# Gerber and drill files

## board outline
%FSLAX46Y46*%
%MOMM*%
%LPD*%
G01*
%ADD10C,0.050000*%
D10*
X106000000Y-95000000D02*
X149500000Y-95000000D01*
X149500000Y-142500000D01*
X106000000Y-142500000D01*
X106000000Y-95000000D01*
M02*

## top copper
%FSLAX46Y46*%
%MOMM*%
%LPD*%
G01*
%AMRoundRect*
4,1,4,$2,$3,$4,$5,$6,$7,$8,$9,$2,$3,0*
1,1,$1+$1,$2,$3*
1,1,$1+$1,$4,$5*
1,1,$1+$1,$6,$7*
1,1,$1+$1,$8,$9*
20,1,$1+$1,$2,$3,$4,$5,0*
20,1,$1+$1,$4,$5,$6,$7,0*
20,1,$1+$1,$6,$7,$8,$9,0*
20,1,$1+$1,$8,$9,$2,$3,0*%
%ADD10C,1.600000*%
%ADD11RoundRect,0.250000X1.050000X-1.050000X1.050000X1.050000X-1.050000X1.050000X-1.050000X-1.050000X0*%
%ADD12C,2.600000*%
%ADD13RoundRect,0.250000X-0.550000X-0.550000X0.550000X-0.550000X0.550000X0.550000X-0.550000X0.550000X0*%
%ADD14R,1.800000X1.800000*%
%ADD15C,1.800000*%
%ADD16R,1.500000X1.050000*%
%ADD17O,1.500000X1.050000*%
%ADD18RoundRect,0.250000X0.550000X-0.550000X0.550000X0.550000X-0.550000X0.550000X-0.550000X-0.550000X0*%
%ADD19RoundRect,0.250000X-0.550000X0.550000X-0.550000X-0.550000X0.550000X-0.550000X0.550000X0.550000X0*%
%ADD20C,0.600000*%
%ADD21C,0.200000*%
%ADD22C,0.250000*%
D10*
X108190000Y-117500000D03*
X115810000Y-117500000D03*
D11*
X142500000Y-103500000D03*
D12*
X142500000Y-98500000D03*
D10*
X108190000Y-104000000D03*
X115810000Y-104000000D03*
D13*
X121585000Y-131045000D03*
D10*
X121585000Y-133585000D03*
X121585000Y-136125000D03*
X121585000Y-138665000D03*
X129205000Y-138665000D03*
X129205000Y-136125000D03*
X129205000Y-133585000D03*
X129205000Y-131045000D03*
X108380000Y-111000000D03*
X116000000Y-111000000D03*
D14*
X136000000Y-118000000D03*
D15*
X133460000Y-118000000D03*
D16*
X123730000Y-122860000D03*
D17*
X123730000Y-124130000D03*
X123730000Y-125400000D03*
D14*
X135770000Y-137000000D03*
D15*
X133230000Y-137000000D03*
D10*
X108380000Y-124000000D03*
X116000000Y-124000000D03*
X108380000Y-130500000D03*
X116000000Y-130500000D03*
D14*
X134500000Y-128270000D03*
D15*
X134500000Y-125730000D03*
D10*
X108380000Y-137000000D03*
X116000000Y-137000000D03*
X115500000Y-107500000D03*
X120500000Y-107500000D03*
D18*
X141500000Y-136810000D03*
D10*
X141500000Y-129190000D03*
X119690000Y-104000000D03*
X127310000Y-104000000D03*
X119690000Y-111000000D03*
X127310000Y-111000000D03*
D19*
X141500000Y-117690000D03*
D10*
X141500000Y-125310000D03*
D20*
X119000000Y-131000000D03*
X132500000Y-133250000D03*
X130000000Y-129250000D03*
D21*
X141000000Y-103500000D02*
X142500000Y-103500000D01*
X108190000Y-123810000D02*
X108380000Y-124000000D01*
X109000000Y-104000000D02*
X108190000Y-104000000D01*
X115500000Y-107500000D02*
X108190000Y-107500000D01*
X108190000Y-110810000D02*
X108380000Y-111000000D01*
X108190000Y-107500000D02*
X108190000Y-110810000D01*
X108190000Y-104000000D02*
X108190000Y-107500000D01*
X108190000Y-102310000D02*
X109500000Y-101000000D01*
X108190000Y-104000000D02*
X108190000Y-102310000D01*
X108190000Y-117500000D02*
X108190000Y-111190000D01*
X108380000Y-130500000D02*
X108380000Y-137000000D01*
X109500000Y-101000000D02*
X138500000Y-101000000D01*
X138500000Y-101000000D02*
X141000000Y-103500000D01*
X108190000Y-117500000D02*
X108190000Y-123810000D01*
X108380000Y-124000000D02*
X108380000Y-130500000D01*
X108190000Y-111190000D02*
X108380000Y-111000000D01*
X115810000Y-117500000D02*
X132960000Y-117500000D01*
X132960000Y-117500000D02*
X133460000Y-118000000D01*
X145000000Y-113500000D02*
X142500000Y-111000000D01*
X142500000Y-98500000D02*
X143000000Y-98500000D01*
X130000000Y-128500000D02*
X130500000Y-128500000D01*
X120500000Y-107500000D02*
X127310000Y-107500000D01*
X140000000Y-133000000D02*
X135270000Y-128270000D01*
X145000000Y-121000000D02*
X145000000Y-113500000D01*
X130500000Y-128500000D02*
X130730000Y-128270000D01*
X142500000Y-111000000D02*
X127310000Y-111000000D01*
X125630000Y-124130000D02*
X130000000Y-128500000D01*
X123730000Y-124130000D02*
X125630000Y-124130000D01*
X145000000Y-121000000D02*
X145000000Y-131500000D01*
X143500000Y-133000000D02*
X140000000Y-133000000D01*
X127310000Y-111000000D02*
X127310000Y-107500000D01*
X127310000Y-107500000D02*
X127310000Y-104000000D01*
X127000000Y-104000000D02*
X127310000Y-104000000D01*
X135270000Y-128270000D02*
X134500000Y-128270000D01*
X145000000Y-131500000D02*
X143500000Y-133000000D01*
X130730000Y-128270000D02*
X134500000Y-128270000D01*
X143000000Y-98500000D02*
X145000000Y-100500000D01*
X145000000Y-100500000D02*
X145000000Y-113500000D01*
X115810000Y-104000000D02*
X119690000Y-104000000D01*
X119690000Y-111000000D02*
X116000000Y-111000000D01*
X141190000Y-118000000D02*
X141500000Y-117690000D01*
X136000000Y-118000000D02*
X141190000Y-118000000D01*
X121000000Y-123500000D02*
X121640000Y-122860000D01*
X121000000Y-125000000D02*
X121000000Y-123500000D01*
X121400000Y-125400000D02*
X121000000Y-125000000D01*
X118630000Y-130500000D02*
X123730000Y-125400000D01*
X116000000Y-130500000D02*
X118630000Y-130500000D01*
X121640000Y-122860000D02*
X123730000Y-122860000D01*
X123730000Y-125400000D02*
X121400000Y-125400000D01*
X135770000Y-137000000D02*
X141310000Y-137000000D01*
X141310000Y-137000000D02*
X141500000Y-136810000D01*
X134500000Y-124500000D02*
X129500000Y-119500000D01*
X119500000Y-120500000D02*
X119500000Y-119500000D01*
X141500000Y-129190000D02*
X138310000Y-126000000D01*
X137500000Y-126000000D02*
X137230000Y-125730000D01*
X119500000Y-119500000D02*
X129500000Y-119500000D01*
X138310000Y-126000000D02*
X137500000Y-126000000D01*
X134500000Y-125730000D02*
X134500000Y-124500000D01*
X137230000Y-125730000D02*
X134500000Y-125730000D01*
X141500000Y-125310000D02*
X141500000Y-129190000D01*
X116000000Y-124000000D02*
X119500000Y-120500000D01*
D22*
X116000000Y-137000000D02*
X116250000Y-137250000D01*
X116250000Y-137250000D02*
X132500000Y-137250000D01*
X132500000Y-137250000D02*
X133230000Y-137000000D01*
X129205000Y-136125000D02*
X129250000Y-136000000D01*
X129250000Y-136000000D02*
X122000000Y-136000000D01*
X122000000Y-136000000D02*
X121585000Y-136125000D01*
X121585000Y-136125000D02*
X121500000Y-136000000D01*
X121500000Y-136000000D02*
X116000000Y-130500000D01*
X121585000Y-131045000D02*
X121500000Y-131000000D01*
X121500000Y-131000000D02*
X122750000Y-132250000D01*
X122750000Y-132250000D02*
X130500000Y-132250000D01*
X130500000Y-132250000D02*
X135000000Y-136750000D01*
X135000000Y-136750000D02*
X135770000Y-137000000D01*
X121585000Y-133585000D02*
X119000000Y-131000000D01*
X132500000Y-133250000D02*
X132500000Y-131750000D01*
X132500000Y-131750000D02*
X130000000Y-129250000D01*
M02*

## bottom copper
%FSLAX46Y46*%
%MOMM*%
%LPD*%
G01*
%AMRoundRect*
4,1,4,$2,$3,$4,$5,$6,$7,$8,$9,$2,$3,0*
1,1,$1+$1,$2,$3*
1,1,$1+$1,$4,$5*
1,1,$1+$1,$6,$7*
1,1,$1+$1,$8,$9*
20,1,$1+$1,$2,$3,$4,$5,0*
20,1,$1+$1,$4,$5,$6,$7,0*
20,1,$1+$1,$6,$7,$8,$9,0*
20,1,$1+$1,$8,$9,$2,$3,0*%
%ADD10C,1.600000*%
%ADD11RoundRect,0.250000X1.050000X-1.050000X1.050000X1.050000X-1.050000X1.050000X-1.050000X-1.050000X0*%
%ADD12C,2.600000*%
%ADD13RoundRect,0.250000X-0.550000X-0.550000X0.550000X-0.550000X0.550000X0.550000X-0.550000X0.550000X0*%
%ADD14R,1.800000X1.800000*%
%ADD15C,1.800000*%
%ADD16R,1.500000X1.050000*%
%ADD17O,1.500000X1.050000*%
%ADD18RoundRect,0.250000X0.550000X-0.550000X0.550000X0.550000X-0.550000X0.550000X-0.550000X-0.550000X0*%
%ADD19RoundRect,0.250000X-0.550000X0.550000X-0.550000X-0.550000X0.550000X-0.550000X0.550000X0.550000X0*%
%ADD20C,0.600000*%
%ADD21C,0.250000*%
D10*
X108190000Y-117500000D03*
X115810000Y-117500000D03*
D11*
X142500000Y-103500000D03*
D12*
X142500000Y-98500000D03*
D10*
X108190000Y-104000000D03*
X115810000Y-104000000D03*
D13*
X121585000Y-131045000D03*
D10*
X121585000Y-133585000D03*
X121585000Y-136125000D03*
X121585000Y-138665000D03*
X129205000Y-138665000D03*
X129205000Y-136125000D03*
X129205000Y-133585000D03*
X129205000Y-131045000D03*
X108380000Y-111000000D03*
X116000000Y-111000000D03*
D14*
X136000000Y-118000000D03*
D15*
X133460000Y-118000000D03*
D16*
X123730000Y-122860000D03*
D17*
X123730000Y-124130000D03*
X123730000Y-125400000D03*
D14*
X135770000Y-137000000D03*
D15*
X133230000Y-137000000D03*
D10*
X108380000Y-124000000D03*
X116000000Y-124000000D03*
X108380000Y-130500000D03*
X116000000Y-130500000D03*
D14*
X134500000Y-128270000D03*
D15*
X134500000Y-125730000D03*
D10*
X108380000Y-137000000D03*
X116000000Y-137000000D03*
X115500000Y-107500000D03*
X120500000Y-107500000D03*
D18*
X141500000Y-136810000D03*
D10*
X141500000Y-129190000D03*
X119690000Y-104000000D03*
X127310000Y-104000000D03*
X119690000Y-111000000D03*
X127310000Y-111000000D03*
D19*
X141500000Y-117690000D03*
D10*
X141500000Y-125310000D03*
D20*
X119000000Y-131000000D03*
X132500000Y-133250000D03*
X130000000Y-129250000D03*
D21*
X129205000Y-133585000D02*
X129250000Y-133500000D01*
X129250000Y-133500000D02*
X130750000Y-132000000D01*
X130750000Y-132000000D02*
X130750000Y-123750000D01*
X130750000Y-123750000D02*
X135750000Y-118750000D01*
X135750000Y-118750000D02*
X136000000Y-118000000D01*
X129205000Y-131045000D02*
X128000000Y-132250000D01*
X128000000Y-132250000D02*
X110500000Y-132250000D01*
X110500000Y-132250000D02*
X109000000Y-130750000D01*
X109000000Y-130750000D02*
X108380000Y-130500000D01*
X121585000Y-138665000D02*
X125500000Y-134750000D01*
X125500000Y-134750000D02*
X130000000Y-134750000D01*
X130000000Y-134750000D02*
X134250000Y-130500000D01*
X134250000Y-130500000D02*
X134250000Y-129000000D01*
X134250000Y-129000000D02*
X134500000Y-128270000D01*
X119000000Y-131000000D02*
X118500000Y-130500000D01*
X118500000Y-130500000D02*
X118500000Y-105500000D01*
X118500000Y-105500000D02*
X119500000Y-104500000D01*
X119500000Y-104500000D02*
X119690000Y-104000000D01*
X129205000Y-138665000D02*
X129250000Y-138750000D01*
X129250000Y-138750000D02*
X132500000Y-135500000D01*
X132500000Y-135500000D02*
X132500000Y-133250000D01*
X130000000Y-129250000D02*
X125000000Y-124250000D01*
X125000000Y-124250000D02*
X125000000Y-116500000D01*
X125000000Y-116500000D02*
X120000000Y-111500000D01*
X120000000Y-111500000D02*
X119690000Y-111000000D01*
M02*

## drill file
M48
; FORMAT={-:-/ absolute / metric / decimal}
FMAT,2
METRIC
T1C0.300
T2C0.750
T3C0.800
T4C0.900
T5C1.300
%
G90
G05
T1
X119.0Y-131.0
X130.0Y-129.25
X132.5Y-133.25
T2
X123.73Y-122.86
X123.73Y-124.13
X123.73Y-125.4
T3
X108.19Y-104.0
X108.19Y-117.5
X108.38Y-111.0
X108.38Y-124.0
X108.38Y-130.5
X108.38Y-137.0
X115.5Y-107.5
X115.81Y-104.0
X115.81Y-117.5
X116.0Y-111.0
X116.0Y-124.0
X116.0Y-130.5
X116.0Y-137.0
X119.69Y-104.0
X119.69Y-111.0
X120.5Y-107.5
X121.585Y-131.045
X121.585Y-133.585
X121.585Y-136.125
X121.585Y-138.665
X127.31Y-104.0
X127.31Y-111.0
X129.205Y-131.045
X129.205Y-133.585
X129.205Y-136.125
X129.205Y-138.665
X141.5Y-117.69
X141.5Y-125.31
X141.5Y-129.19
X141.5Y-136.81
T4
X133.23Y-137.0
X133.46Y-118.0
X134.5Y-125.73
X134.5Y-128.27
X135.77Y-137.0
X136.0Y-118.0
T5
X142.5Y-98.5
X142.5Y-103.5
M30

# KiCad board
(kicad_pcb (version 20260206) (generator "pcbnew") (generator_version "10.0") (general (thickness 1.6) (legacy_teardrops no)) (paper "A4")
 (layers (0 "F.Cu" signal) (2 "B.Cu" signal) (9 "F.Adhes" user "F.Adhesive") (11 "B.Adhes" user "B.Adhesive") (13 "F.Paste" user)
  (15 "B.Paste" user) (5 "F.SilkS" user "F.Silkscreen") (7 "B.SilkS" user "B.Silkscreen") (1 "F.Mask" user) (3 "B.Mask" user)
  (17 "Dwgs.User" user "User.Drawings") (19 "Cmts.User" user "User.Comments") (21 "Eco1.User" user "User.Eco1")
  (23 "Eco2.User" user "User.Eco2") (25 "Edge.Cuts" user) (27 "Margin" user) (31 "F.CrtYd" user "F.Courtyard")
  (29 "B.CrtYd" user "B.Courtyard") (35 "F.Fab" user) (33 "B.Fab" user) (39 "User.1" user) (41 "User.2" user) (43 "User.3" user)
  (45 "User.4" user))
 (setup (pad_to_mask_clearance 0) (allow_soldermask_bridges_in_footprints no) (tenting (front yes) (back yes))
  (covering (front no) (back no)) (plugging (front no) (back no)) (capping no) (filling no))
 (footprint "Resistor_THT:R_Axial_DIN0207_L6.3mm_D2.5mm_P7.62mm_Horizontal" (layer "F.Cu") (at 108.19 117.5)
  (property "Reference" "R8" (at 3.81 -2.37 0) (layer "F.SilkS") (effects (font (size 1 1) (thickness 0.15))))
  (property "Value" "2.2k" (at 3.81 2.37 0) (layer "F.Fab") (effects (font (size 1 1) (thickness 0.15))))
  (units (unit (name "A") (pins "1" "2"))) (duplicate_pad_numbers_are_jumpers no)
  (pad "1" thru_hole circle (at 0 0) (size 1.6 1.6) (drill 0.8) (layers "*.Cu" "*.Mask") (remove_unused_layers no) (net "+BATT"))
  (pad "2" thru_hole circle (at 7.62 0) (size 1.6 1.6) (drill 0.8) (layers "*.Cu" "*.Mask") (remove_unused_layers no) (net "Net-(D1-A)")))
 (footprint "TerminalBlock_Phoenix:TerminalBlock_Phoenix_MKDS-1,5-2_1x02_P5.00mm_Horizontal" (layer "F.Cu") (at 142.5 103.5 90)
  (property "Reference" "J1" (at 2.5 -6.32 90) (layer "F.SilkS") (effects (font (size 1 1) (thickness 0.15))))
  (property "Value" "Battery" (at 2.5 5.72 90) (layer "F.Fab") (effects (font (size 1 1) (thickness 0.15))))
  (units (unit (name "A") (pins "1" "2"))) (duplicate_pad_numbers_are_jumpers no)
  (pad "1" thru_hole roundrect (at 0 0 90) (size 2.6 2.6) (drill 1.3) (layers "*.Cu" "*.Mask") (remove_unused_layers no)
   (roundrect_rratio 0.096154) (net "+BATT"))
  (pad "2" thru_hole circle (at 5 0 90) (size 2.6 2.6) (drill 1.3) (layers "*.Cu" "*.Mask") (remove_unused_layers no) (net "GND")))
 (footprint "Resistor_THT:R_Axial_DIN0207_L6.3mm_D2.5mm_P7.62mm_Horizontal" (layer "F.Cu") (at 108.19 104)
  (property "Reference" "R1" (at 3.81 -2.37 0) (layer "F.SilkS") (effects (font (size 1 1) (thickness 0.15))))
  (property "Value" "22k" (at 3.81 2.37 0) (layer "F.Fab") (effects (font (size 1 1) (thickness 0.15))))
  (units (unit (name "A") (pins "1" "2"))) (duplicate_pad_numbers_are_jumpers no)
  (pad "1" thru_hole circle (at 0 0) (size 1.6 1.6) (drill 0.8) (layers "*.Cu" "*.Mask") (remove_unused_layers no) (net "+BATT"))
  (pad "2" thru_hole circle (at 7.62 0) (size 1.6 1.6) (drill 0.8) (layers "*.Cu" "*.Mask") (remove_unused_layers no) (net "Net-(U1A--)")))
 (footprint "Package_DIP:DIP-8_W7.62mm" (layer "F.Cu") (at 121.585 131.045)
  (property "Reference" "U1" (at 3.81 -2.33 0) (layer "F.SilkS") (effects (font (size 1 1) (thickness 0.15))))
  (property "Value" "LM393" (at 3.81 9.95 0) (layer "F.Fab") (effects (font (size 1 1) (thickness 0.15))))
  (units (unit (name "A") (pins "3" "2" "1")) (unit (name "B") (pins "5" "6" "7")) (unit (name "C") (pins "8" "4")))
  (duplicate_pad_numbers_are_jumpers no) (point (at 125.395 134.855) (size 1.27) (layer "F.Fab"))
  (pad "1" thru_hole roundrect (at 0 0) (size 1.6 1.6) (drill 0.8) (layers "*.Cu" "*.Mask") (remove_unused_layers no)
   (roundrect_rratio 0.15625) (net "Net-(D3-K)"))
  (pad "2" thru_hole circle (at 0 2.54) (size 1.6 1.6) (drill 0.8) (layers "*.Cu" "*.Mask") (remove_unused_layers no) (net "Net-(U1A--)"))
  (pad "3" thru_hole circle (at 0 5.08) (size 1.6 1.6) (drill 0.8) (layers "*.Cu" "*.Mask") (remove_unused_layers no) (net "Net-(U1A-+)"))
  (pad "4" thru_hole circle (at 0 7.62) (size 1.6 1.6) (drill 0.8) (layers "*.Cu" "*.Mask") (remove_unused_layers no) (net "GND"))
  (pad "5" thru_hole circle (at 7.62 7.62) (size 1.6 1.6) (drill 0.8) (layers "*.Cu" "*.Mask") (remove_unused_layers no) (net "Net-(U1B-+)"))
  (pad "6" thru_hole circle (at 7.62 5.08) (size 1.6 1.6) (drill 0.8) (layers "*.Cu" "*.Mask") (remove_unused_layers no) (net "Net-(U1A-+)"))
  (pad "7" thru_hole circle (at 7.62 2.54) (size 1.6 1.6) (drill 0.8) (layers "*.Cu" "*.Mask") (remove_unused_layers no) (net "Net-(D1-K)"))
  (pad "8" thru_hole circle (at 7.62 0) (size 1.6 1.6) (drill 0.8) (layers "*.Cu" "*.Mask") (remove_unused_layers no) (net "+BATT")))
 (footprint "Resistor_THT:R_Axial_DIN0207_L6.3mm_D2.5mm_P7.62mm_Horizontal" (layer "F.Cu") (at 108.38 111)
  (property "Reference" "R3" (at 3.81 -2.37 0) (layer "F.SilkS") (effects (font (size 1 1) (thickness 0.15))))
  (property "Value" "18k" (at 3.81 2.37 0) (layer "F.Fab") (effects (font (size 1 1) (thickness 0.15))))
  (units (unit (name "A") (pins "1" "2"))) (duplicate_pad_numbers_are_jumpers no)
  (pad "1" thru_hole circle (at 0 0) (size 1.6 1.6) (drill 0.8) (layers "*.Cu" "*.Mask") (remove_unused_layers no) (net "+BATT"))
  (pad "2" thru_hole circle (at 7.62 0) (size 1.6 1.6) (drill 0.8) (layers "*.Cu" "*.Mask") (remove_unused_layers no) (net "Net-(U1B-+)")))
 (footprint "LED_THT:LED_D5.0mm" (layer "F.Cu") (at 136 118 180)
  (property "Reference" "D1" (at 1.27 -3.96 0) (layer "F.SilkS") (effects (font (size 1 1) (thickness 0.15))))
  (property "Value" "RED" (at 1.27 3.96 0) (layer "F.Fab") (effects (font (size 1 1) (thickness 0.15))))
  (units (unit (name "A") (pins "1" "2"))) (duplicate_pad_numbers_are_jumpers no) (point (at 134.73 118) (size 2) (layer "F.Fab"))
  (pad "1" thru_hole rect (at 0 0 180) (size 1.8 1.8) (drill 0.9) (layers "*.Cu" "*.Mask") (remove_unused_layers no) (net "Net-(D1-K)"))
  (pad "2" thru_hole circle (at 2.54 0 180) (size 1.8 1.8) (drill 0.9) (layers "*.Cu" "*.Mask") (remove_unused_layers no) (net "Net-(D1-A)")))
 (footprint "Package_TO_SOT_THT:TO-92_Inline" (layer "F.Cu") (at 123.73 122.86 -90)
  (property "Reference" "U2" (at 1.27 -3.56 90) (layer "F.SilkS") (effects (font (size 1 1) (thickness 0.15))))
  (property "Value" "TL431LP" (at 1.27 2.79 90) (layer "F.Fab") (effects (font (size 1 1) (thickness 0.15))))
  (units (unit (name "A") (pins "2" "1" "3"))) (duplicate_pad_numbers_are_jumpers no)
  (pad "1" thru_hole rect (at 0 0 270) (size 1.05 1.5) (drill 0.75) (layers "*.Cu" "*.Mask") (remove_unused_layers no) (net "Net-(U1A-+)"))
  (pad "2" thru_hole oval (at 1.27 0 270) (size 1.05 1.5) (drill 0.75) (layers "*.Cu" "*.Mask") (remove_unused_layers no) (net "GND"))
  (pad "3" thru_hole oval (at 2.54 0 270) (size 1.05 1.5) (drill 0.75) (layers "*.Cu" "*.Mask") (remove_unused_layers no)
   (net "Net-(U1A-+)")))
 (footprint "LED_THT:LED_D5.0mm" (layer "F.Cu") (at 135.77 137 180)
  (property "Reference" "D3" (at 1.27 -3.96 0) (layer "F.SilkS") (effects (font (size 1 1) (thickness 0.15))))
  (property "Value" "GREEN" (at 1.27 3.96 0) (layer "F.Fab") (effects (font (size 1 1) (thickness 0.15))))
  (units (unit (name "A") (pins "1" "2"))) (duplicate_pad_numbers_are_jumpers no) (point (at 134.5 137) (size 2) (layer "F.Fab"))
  (pad "1" thru_hole rect (at 0 0 180) (size 1.8 1.8) (drill 0.9) (layers "*.Cu" "*.Mask") (remove_unused_layers no) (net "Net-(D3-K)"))
  (pad "2" thru_hole circle (at 2.54 0 180) (size 1.8 1.8) (drill 0.9) (layers "*.Cu" "*.Mask") (remove_unused_layers no) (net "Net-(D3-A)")))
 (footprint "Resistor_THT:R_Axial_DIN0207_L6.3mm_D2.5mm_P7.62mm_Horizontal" (layer "F.Cu") (at 108.38 124)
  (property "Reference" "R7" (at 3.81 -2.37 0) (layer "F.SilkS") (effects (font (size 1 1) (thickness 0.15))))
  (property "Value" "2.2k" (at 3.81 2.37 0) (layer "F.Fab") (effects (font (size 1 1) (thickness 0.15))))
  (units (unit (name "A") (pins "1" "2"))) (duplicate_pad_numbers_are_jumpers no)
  (pad "1" thru_hole circle (at 0 0) (size 1.6 1.6) (drill 0.8) (layers "*.Cu" "*.Mask") (remove_unused_layers no) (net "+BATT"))
  (pad "2" thru_hole circle (at 7.62 0) (size 1.6 1.6) (drill 0.8) (layers "*.Cu" "*.Mask") (remove_unused_layers no) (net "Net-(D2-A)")))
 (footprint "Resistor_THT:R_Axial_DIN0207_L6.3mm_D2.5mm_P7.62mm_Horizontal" (layer "F.Cu") (at 108.38 130.5)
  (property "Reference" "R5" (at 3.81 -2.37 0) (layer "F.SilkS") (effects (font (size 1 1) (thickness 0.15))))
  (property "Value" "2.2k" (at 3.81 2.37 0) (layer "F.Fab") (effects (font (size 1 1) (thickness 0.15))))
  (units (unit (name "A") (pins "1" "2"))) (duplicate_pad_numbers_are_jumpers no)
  (pad "1" thru_hole circle (at 0 0) (size 1.6 1.6) (drill 0.8) (layers "*.Cu" "*.Mask") (remove_unused_layers no) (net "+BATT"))
  (pad "2" thru_hole circle (at 7.62 0) (size 1.6 1.6) (drill 0.8) (layers "*.Cu" "*.Mask") (remove_unused_layers no) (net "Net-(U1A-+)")))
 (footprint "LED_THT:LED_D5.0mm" (layer "F.Cu") (at 134.5 128.27 90)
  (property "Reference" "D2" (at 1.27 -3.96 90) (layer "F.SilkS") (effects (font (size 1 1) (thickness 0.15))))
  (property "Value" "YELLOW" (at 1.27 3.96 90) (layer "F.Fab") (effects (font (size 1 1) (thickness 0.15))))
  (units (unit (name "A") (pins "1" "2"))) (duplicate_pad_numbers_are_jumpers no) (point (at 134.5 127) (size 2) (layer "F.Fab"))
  (pad "1" thru_hole rect (at 0 0 90) (size 1.8 1.8) (drill 0.9) (layers "*.Cu" "*.Mask") (remove_unused_layers no) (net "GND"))
  (pad "2" thru_hole circle (at 2.54 0 90) (size 1.8 1.8) (drill 0.9) (layers "*.Cu" "*.Mask") (remove_unused_layers no) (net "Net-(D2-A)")))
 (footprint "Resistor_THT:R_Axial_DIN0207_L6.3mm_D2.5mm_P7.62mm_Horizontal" (layer "F.Cu") (at 108.38 137)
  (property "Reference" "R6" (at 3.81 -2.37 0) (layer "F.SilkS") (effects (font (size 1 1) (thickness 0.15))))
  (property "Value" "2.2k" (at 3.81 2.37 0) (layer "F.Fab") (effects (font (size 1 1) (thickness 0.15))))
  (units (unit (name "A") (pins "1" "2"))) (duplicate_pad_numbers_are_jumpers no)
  (pad "1" thru_hole circle (at 0 0) (size 1.6 1.6) (drill 0.8) (layers "*.Cu" "*.Mask") (remove_unused_layers no) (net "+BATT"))
  (pad "2" thru_hole circle (at 7.62 0) (size 1.6 1.6) (drill 0.8) (layers "*.Cu" "*.Mask") (remove_unused_layers no) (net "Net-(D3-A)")))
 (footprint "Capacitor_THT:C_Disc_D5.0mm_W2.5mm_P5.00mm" (layer "F.Cu") (at 115.5 107.5)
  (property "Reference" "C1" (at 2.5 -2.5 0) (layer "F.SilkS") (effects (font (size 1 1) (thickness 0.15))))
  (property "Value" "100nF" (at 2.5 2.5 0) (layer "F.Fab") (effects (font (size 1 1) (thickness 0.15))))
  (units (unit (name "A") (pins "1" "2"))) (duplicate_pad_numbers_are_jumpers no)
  (pad "1" thru_hole circle (at 0 0) (size 1.6 1.6) (drill 0.8) (layers "*.Cu" "*.Mask") (remove_unused_layers no) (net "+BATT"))
  (pad "2" thru_hole circle (at 5 0) (size 1.6 1.6) (drill 0.8) (layers "*.Cu" "*.Mask") (remove_unused_layers no) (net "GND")))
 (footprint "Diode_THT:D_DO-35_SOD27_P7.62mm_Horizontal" (layer "F.Cu") (at 141.5 136.81 90)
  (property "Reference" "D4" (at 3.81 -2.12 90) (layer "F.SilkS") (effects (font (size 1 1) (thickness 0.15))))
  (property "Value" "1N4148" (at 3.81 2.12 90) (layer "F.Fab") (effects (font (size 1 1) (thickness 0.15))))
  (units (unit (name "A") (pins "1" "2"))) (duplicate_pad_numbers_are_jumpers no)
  (pad "1" thru_hole roundrect (at 0 0 90) (size 1.6 1.6) (drill 0.8) (layers "*.Cu" "*.Mask") (remove_unused_layers no)
   (roundrect_rratio 0.15625) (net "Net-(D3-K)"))
  (pad "2" thru_hole circle (at 7.62 0 90) (size 1.6 1.6) (drill 0.8) (layers "*.Cu" "*.Mask") (remove_unused_layers no) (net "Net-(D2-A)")))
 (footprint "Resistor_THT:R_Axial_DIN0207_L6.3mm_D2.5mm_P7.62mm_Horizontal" (layer "F.Cu") (at 119.69 104)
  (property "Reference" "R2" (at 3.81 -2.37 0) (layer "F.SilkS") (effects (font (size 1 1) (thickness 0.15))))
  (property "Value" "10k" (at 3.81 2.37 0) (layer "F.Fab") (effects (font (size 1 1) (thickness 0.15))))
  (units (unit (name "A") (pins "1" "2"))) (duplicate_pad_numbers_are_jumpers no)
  (pad "1" thru_hole circle (at 0 0) (size 1.6 1.6) (drill 0.8) (layers "*.Cu" "*.Mask") (remove_unused_layers no) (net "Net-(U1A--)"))
  (pad "2" thru_hole circle (at 7.62 0) (size 1.6 1.6) (drill 0.8) (layers "*.Cu" "*.Mask") (remove_unused_layers no) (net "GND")))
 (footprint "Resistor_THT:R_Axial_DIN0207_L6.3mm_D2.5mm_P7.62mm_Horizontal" (layer "F.Cu") (at 119.69 111)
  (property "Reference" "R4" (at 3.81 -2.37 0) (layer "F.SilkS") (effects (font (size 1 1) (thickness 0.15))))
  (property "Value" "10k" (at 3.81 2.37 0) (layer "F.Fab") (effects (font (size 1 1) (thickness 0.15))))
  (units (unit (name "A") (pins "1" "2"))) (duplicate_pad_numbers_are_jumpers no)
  (pad "1" thru_hole circle (at 0 0) (size 1.6 1.6) (drill 0.8) (layers "*.Cu" "*.Mask") (remove_unused_layers no) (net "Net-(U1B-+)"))
  (pad "2" thru_hole circle (at 7.62 0) (size 1.6 1.6) (drill 0.8) (layers "*.Cu" "*.Mask") (remove_unused_layers no) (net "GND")))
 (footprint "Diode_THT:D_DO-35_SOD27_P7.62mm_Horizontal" (layer "F.Cu") (at 141.5 117.69 -90)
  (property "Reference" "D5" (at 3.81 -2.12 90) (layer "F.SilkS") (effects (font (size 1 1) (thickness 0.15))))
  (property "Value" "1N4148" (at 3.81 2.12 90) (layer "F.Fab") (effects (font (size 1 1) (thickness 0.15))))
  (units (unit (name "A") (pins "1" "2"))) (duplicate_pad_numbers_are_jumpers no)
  (pad "1" thru_hole roundrect (at 0 0 270) (size 1.6 1.6) (drill 0.8) (layers "*.Cu" "*.Mask") (remove_unused_layers no)
   (roundrect_rratio 0.15625) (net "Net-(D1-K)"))
  (pad "2" thru_hole circle (at 7.62 0 270) (size 1.6 1.6) (drill 0.8) (layers "*.Cu" "*.Mask") (remove_unused_layers no) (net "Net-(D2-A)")))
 (gr_rect (start 106 95) (end 149.5 142.5) (stroke (width 0.05) (type default)) (fill no) (layer "Edge.Cuts"))
 (segment (start 141 103.5) (end 142.5 103.5) (width 0.2) (layer "F.Cu") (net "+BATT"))
 (segment (start 108.19 123.81) (end 108.38 124) (width 0.2) (layer "F.Cu") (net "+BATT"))
 (segment (start 109 104) (end 108.19 104) (width 0.2) (layer "F.Cu") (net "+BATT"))
 (segment (start 115.5 107.5) (end 108.19 107.5) (width 0.2) (layer "F.Cu") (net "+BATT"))
 (segment (start 108.19 110.81) (end 108.38 111) (width 0.2) (layer "F.Cu") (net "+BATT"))
 (segment (start 108.19 107.5) (end 108.19 110.81) (width 0.2) (layer "F.Cu") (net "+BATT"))
 (segment (start 108.19 104) (end 108.19 107.5) (width 0.2) (layer "F.Cu") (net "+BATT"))
 (segment (start 108.19 102.31) (end 109.5 101) (width 0.2) (layer "F.Cu") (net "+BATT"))
 (segment (start 108.19 104) (end 108.19 102.31) (width 0.2) (layer "F.Cu") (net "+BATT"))
 (segment (start 108.19 117.5) (end 108.19 111.19) (width 0.2) (layer "F.Cu") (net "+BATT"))
 (segment (start 108.38 130.5) (end 108.38 137) (width 0.2) (layer "F.Cu") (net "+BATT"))
 (segment (start 109.5 101) (end 138.5 101) (width 0.2) (layer "F.Cu") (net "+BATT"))
 (segment (start 138.5 101) (end 141 103.5) (width 0.2) (layer "F.Cu") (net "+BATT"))
 (segment (start 108.19 117.5) (end 108.19 123.81) (width 0.2) (layer "F.Cu") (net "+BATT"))
 (segment (start 108.38 124) (end 108.38 130.5) (width 0.2) (layer "F.Cu") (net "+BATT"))
 (segment (start 108.19 111.19) (end 108.38 111) (width 0.2) (layer "F.Cu") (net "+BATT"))
 (segment (start 115.81 117.5) (end 132.96 117.5) (width 0.2) (layer "F.Cu") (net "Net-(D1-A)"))
 (segment (start 132.96 117.5) (end 133.46 118) (width 0.2) (layer "F.Cu") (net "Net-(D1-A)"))
 (segment (start 145 113.5) (end 142.5 111) (width 0.2) (layer "F.Cu") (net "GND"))
 (segment (start 142.5 98.5) (end 143 98.5) (width 0.2) (layer "F.Cu") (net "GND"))
 (segment (start 130 128.5) (end 130.5 128.5) (width 0.2) (layer "F.Cu") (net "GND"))
 (segment (start 120.5 107.5) (end 127.31 107.5) (width 0.2) (layer "F.Cu") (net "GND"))
 (segment (start 140 133) (end 135.27 128.27) (width 0.2) (layer "F.Cu") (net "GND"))
 (segment (start 145 121) (end 145 113.5) (width 0.2) (layer "F.Cu") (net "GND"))
 (segment (start 130.5 128.5) (end 130.73 128.27) (width 0.2) (layer "F.Cu") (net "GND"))
 (segment (start 142.5 111) (end 127.31 111) (width 0.2) (layer "F.Cu") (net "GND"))
 (segment (start 125.63 124.13) (end 130 128.5) (width 0.2) (layer "F.Cu") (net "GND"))
 (segment (start 123.73 124.13) (end 125.63 124.13) (width 0.2) (layer "F.Cu") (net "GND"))
 (segment (start 145 121) (end 145 131.5) (width 0.2) (layer "F.Cu") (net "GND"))
 (segment (start 143.5 133) (end 140 133) (width 0.2) (layer "F.Cu") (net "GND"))
 (segment (start 127.31 111) (end 127.31 107.5) (width 0.2) (layer "F.Cu") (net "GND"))
 (segment (start 127.31 107.5) (end 127.31 104) (width 0.2) (layer "F.Cu") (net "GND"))
 (segment (start 127 104) (end 127.31 104) (width 0.2) (layer "F.Cu") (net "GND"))
 (segment (start 135.27 128.27) (end 134.5 128.27) (width 0.2) (layer "F.Cu") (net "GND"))
 (segment (start 145 131.5) (end 143.5 133) (width 0.2) (layer "F.Cu") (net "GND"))
 (segment (start 130.73 128.27) (end 134.5 128.27) (width 0.2) (layer "F.Cu") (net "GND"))
 (segment (start 143 98.5) (end 145 100.5) (width 0.2) (layer "F.Cu") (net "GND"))
 (segment (start 145 100.5) (end 145 113.5) (width 0.2) (layer "F.Cu") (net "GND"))
 (segment (start 115.81 104) (end 119.69 104) (width 0.2) (layer "F.Cu") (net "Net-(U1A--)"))
 (segment (start 119.69 111) (end 116 111) (width 0.2) (layer "F.Cu") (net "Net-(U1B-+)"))
 (segment (start 141.19 118) (end 141.5 117.69) (width 0.2) (layer "F.Cu") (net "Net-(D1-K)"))
 (segment (start 136 118) (end 141.19 118) (width 0.2) (layer "F.Cu") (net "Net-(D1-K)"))
 (segment (start 121 123.5) (end 121.64 122.86) (width 0.2) (layer "F.Cu") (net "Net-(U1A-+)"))
 (segment (start 121 125) (end 121 123.5) (width 0.2) (layer "F.Cu") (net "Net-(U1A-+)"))
 (segment (start 121.4 125.4) (end 121 125) (width 0.2) (layer "F.Cu") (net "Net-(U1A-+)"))
 (segment (start 118.63 130.5) (end 123.73 125.4) (width 0.2) (layer "F.Cu") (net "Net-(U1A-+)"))
 (segment (start 116 130.5) (end 118.63 130.5) (width 0.2) (layer "F.Cu") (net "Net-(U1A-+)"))
 (segment (start 121.64 122.86) (end 123.73 122.86) (width 0.2) (layer "F.Cu") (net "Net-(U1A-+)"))
 (segment (start 123.73 125.4) (end 121.4 125.4) (width 0.2) (layer "F.Cu") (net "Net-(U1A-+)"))
 (segment (start 135.77 137) (end 141.31 137) (width 0.2) (layer "F.Cu") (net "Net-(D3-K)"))
 (segment (start 141.31 137) (end 141.5 136.81) (width 0.2) (layer "F.Cu") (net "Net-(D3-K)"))
 (segment (start 134.5 124.5) (end 129.5 119.5) (width 0.2) (layer "F.Cu") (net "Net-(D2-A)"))
 (segment (start 119.5 120.5) (end 119.5 119.5) (width 0.2) (layer "F.Cu") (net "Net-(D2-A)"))
 (segment (start 141.5 129.19) (end 138.31 126) (width 0.2) (layer "F.Cu") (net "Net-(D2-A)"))
 (segment (start 137.5 126) (end 137.23 125.73) (width 0.2) (layer "F.Cu") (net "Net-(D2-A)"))
 (segment (start 119.5 119.5) (end 129.5 119.5) (width 0.2) (layer "F.Cu") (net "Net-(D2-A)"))
 (segment (start 138.31 126) (end 137.5 126) (width 0.2) (layer "F.Cu") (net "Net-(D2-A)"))
 (segment (start 134.5 125.73) (end 134.5 124.5) (width 0.2) (layer "F.Cu") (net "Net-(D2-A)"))
 (segment (start 137.23 125.73) (end 134.5 125.73) (width 0.2) (layer "F.Cu") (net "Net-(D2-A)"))
 (segment (start 141.5 125.31) (end 141.5 129.19) (width 0.2) (layer "F.Cu") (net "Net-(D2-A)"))
 (segment (start 116 124) (end 119.5 120.5) (width 0.2) (layer "F.Cu") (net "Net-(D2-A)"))
 (segment (start 116 137) (end 116.25 137.25) (width 0.25) (layer "F.Cu") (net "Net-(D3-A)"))
 (segment (start 116.25 137.25) (end 132.5 137.25) (width 0.25) (layer "F.Cu") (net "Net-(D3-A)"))
 (segment (start 132.5 137.25) (end 133.23 137) (width 0.25) (layer "F.Cu") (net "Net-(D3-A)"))
 (segment (start 129.205 136.125) (end 129.25 136) (width 0.25) (layer "F.Cu") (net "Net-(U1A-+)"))
 (segment (start 129.25 136) (end 122 136) (width 0.25) (layer "F.Cu") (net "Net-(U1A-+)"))
 (segment (start 122 136) (end 121.585 136.125) (width 0.25) (layer "F.Cu") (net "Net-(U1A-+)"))
 (segment (start 121.585 136.125) (end 121.5 136) (width 0.25) (layer "F.Cu") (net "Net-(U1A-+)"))
 (segment (start 121.5 136) (end 116 130.5) (width 0.25) (layer "F.Cu") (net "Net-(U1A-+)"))
 (segment (start 121.585 131.045) (end 121.5 131) (width 0.25) (layer "F.Cu") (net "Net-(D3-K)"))
 (segment (start 121.5 131) (end 122.75 132.25) (width 0.25) (layer "F.Cu") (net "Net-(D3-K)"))
 (segment (start 122.75 132.25) (end 130.5 132.25) (width 0.25) (layer "F.Cu") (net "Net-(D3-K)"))
 (segment (start 130.5 132.25) (end 135 136.75) (width 0.25) (layer "F.Cu") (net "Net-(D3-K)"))
 (segment (start 135 136.75) (end 135.77 137) (width 0.25) (layer "F.Cu") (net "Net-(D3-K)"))
 (segment (start 129.205 133.585) (end 129.25 133.5) (width 0.25) (layer "B.Cu") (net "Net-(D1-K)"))
 (segment (start 129.25 133.5) (end 130.75 132) (width 0.25) (layer "B.Cu") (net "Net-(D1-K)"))
 (segment (start 130.75 132) (end 130.75 123.75) (width 0.25) (layer "B.Cu") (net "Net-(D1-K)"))
 (segment (start 130.75 123.75) (end 135.75 118.75) (width 0.25) (layer "B.Cu") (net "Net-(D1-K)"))
 (segment (start 135.75 118.75) (end 136 118) (width 0.25) (layer "B.Cu") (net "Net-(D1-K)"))
 (segment (start 129.205 131.045) (end 128 132.25) (width 0.25) (layer "B.Cu") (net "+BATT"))
 (segment (start 128 132.25) (end 110.5 132.25) (width 0.25) (layer "B.Cu") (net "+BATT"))
 (segment (start 110.5 132.25) (end 109 130.75) (width 0.25) (layer "B.Cu") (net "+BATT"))
 (segment (start 109 130.75) (end 108.38 130.5) (width 0.25) (layer "B.Cu") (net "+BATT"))
 (segment (start 121.585 138.665) (end 125.5 134.75) (width 0.25) (layer "B.Cu") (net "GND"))
 (segment (start 125.5 134.75) (end 130 134.75) (width 0.25) (layer "B.Cu") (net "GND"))
 (segment (start 130 134.75) (end 134.25 130.5) (width 0.25) (layer "B.Cu") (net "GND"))
 (segment (start 134.25 130.5) (end 134.25 129) (width 0.25) (layer "B.Cu") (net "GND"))
 (segment (start 134.25 129) (end 134.5 128.27) (width 0.25) (layer "B.Cu") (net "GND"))
 (segment (start 121.585 133.585) (end 119 131) (width 0.25) (layer "F.Cu") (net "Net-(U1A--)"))
 (segment (start 119 131) (end 118.5 130.5) (width 0.25) (layer "B.Cu") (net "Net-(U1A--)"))
 (segment (start 118.5 130.5) (end 118.5 105.5) (width 0.25) (layer "B.Cu") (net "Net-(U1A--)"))
 (segment (start 118.5 105.5) (end 119.5 104.5) (width 0.25) (layer "B.Cu") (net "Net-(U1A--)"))
 (segment (start 119.5 104.5) (end 119.69 104) (width 0.25) (layer "B.Cu") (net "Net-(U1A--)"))
 (segment (start 129.205 138.665) (end 129.25 138.75) (width 0.25) (layer "B.Cu") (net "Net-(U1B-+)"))
 (segment (start 129.25 138.75) (end 132.5 135.5) (width 0.25) (layer "B.Cu") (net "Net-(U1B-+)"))
 (segment (start 132.5 135.5) (end 132.5 133.25) (width 0.25) (layer "B.Cu") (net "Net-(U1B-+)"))
 (segment (start 132.5 133.25) (end 132.5 131.75) (width 0.25) (layer "F.Cu") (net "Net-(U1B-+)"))
 (segment (start 132.5 131.75) (end 130 129.25) (width 0.25) (layer "F.Cu") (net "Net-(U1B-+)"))
 (segment (start 130 129.25) (end 125 124.25) (width 0.25) (layer "B.Cu") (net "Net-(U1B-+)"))
 (segment (start 125 124.25) (end 125 116.5) (width 0.25) (layer "B.Cu") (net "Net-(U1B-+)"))
 (segment (start 125 116.5) (end 120 111.5) (width 0.25) (layer "B.Cu") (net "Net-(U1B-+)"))
 (segment (start 120 111.5) (end 119.69 111) (width 0.25) (layer "B.Cu") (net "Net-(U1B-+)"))
 (via (at 119 131) (size 0.6) (drill 0.3) (layers "F.Cu" "B.Cu") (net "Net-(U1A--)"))
 (via (at 132.5 133.25) (size 0.6) (drill 0.3) (layers "F.Cu" "B.Cu") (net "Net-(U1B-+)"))
 (via (at 130 129.25) (size 0.6) (drill 0.3) (layers "F.Cu" "B.Cu") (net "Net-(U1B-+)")))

